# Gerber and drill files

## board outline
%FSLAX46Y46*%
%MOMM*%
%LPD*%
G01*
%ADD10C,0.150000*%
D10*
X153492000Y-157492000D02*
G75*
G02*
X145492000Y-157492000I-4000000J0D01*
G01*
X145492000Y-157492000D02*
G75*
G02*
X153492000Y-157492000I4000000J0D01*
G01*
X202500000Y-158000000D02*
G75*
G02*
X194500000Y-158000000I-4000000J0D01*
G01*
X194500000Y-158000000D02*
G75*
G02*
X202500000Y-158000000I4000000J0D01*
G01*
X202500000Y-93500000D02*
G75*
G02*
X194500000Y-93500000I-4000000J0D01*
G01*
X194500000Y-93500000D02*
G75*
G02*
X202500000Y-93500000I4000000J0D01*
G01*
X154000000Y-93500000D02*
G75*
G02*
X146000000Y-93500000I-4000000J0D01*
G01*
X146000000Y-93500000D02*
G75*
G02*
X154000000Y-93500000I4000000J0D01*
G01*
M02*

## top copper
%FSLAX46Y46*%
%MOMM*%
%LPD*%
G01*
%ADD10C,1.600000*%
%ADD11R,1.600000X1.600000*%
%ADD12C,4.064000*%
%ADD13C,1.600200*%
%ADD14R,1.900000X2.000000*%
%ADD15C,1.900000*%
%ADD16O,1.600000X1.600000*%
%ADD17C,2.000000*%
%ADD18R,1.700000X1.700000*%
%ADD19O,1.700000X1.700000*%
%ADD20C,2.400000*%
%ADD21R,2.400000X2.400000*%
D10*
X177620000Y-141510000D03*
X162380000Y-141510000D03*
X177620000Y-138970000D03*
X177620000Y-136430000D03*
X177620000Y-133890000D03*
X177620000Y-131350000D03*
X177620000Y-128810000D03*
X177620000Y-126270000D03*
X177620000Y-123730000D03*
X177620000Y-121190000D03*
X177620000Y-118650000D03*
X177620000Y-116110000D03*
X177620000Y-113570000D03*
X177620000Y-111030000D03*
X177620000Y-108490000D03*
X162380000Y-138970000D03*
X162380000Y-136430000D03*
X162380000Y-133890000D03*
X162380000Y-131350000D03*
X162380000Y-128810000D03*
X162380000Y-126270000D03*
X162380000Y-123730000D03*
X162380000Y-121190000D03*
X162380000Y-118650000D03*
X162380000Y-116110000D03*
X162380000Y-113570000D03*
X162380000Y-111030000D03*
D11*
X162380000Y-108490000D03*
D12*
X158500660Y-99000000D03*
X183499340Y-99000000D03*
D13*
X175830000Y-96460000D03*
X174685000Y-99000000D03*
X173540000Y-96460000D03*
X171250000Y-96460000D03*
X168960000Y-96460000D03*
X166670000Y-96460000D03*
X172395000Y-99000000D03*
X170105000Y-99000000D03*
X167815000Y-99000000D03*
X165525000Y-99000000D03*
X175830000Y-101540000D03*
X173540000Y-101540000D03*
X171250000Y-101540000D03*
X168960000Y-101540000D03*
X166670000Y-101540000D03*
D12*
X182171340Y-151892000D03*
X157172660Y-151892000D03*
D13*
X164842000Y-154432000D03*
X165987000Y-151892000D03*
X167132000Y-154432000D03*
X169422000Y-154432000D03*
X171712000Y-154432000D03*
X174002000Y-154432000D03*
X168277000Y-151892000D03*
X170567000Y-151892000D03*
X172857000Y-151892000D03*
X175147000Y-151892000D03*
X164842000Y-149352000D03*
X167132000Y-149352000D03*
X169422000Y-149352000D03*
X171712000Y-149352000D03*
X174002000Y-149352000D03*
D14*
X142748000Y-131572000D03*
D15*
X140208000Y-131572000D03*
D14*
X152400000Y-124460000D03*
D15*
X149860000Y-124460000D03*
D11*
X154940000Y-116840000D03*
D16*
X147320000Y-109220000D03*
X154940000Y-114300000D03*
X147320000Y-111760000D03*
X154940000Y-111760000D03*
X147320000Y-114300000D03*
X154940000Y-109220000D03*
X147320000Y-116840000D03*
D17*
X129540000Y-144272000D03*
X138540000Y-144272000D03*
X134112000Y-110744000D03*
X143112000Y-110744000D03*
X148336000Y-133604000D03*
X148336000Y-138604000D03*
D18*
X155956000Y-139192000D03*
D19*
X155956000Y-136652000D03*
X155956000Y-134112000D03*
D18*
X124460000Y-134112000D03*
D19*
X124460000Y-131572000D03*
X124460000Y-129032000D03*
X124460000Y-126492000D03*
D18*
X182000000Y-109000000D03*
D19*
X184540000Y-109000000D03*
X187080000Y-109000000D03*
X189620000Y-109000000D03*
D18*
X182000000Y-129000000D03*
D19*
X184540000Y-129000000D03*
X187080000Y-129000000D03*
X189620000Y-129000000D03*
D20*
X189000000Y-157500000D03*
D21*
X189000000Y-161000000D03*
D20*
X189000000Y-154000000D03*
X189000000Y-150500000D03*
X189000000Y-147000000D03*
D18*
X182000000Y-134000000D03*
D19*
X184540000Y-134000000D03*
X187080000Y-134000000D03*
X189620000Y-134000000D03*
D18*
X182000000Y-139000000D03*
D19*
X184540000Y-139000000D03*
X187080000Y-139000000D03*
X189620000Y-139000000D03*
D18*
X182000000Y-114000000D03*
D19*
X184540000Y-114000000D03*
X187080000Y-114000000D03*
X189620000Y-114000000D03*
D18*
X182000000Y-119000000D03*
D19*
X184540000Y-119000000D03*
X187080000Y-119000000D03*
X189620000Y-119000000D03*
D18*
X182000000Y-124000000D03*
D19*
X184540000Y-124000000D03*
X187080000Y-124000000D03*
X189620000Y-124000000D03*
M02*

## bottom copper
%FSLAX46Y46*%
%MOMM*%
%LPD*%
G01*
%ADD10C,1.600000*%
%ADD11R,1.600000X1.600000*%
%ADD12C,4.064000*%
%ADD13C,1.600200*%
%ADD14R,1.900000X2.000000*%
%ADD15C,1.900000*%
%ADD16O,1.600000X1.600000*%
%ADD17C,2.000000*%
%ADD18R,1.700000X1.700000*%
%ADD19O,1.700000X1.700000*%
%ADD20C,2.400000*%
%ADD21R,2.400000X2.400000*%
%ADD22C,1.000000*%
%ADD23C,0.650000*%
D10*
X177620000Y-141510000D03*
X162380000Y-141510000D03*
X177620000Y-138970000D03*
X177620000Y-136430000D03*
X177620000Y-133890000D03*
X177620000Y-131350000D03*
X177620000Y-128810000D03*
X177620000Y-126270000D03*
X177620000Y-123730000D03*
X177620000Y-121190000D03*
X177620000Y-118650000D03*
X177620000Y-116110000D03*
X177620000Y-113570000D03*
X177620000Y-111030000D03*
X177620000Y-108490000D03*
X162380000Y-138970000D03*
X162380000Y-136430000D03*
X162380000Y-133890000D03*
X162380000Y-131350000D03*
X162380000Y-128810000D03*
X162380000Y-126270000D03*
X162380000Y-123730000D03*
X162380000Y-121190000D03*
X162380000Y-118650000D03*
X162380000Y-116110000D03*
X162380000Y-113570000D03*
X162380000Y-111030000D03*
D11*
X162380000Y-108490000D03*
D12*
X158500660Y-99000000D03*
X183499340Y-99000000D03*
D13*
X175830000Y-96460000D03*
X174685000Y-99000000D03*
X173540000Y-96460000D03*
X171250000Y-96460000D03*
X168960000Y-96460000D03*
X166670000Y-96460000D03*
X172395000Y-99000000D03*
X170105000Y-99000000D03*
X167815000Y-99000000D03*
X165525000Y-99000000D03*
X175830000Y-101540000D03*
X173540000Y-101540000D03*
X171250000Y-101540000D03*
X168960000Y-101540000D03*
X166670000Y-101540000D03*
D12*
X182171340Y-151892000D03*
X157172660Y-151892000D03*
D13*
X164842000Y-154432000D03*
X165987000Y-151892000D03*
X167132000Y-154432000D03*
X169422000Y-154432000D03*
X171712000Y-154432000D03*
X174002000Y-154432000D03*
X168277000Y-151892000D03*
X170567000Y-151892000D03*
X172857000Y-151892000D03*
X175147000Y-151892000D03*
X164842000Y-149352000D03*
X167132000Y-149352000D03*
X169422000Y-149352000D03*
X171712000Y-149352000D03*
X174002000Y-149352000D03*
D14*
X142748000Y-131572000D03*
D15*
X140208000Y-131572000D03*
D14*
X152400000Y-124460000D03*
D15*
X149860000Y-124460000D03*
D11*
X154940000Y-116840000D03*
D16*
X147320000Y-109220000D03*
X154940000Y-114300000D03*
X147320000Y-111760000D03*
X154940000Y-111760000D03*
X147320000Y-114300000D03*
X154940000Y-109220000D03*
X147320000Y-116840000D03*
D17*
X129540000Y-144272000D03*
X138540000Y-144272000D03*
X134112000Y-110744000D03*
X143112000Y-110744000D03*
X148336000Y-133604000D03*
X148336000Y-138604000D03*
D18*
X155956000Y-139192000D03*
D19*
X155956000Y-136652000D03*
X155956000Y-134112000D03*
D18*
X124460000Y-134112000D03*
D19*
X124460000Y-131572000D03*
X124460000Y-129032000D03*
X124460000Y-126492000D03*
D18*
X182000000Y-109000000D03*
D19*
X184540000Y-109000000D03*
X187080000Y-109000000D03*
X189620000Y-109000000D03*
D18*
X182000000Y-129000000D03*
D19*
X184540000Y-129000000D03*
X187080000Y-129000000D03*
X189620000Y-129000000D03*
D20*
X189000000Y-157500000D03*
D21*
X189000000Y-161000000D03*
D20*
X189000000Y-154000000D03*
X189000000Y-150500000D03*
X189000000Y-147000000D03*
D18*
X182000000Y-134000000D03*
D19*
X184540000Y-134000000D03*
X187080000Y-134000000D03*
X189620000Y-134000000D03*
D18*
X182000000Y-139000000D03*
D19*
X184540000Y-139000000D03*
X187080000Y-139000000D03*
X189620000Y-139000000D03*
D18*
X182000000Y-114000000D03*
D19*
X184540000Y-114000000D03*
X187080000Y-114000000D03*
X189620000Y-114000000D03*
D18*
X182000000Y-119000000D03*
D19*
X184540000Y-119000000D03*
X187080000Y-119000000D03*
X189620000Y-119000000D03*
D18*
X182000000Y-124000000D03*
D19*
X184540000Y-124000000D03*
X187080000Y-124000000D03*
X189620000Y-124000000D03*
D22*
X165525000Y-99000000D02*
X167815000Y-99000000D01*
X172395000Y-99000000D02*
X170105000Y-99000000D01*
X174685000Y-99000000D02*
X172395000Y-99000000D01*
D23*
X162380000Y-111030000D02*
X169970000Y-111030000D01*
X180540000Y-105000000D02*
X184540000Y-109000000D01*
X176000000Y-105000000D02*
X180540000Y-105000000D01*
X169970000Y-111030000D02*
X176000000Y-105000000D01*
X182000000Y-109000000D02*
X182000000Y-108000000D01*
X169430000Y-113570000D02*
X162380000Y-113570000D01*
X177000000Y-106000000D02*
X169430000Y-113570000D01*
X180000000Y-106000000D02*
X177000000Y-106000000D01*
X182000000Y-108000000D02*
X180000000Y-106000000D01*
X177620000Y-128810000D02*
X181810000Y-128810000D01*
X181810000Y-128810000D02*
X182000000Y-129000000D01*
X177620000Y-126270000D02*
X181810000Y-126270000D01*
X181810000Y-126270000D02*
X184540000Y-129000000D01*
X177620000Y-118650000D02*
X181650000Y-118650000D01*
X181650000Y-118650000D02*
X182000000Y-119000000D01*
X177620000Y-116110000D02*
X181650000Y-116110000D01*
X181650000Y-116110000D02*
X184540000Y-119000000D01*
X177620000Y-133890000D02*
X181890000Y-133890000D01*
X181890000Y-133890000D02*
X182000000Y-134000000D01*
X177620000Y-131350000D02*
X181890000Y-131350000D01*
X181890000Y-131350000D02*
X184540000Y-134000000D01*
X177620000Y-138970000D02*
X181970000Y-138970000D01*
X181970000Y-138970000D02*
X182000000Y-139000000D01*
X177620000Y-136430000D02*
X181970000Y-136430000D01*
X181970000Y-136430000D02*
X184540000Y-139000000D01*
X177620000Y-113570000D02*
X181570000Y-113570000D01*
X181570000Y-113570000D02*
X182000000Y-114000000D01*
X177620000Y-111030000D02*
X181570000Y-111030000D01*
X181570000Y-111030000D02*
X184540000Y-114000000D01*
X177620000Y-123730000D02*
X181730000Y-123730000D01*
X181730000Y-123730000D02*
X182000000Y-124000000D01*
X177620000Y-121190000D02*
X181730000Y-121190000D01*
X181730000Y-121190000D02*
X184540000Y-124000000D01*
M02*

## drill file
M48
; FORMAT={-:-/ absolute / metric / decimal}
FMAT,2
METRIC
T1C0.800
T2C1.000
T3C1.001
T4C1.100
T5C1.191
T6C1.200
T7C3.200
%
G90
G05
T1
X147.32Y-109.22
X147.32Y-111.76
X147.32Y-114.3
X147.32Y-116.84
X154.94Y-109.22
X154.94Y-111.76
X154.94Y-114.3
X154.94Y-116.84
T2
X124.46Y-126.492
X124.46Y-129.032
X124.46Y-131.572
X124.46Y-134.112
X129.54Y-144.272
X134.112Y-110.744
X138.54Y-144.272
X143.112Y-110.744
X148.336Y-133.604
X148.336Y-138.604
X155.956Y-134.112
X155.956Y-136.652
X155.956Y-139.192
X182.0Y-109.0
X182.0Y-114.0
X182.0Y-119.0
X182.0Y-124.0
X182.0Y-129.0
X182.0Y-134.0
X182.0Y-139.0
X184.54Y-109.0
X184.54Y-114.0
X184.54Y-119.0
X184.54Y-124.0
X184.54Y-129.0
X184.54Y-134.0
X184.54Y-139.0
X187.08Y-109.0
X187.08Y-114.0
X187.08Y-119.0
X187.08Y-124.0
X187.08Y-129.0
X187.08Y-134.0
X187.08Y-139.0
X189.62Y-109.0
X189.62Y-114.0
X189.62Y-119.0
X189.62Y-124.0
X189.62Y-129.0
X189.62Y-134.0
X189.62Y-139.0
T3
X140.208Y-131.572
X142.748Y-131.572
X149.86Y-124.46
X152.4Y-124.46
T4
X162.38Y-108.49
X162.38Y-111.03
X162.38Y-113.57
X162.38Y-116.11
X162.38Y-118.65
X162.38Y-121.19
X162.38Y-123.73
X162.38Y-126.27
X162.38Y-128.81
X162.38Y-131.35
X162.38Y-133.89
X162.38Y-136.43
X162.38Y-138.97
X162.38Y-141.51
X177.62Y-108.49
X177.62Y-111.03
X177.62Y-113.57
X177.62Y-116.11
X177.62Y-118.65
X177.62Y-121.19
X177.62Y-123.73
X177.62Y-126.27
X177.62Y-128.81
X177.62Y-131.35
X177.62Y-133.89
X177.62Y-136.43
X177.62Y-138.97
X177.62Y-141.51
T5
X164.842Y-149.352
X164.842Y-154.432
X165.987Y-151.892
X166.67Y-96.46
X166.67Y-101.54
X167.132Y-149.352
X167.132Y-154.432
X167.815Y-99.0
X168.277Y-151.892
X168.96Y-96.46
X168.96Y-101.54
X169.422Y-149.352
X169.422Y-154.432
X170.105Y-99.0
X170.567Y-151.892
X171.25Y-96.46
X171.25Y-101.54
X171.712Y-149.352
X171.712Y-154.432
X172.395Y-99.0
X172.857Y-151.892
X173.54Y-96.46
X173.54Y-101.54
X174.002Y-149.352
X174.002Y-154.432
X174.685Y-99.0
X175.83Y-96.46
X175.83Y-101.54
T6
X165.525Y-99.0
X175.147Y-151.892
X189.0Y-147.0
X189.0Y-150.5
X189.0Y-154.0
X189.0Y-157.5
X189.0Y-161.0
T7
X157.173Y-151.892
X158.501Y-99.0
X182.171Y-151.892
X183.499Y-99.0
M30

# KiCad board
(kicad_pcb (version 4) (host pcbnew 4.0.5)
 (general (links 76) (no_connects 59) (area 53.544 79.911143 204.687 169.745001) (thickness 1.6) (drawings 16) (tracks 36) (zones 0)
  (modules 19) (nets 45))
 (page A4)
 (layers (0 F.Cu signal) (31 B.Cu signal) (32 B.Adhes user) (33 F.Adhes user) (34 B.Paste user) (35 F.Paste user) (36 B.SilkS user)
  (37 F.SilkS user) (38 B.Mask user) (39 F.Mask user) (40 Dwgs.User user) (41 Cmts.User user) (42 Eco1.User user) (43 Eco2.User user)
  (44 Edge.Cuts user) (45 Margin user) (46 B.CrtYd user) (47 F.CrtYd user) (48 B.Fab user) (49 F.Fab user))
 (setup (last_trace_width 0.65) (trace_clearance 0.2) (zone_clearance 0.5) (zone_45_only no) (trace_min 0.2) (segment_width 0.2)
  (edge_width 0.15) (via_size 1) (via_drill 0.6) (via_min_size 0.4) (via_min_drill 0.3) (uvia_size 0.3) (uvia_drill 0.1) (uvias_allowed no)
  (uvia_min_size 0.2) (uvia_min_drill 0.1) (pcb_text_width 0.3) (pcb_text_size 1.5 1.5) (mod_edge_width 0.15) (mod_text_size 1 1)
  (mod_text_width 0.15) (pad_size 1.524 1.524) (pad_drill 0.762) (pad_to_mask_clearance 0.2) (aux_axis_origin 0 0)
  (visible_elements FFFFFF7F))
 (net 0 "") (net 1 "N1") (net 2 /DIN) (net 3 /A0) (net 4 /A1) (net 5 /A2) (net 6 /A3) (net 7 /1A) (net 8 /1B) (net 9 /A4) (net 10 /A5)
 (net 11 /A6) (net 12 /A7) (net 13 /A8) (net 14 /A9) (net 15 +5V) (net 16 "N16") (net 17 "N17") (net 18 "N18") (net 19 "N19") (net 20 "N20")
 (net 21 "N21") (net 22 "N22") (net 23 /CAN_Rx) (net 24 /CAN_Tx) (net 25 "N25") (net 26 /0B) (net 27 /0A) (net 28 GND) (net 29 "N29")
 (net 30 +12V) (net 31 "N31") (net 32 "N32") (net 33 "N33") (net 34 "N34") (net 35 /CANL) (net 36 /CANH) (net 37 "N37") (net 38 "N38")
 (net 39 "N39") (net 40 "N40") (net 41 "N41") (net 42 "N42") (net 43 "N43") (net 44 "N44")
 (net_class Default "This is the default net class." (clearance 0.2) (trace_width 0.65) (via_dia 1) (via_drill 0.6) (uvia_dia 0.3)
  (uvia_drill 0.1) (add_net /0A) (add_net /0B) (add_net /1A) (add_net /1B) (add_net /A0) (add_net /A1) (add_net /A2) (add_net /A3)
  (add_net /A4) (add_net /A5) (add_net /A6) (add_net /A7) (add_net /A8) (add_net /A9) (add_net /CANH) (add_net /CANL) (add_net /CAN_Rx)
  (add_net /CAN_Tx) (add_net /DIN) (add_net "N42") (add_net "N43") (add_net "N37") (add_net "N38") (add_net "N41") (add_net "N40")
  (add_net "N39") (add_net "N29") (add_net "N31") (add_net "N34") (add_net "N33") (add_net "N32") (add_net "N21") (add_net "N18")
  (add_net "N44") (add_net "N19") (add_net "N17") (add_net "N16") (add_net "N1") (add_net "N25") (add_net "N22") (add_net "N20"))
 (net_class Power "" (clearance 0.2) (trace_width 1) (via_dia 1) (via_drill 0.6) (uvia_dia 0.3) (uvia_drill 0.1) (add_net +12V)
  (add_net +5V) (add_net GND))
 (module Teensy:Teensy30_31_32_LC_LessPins (layer F.Cu) (at 170 125 270)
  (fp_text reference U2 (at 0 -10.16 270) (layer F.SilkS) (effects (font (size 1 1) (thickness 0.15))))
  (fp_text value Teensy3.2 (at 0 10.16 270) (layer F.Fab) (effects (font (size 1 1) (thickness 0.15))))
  (pad 20 thru_hole circle (at 16.51 -7.62 270) (size 1.6 1.6) (drill 1.1) (layers *.Cu *.Mask F.SilkS) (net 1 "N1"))
  (pad 14 thru_hole circle (at 16.51 7.62 270) (size 1.6 1.6) (drill 1.1) (layers *.Cu *.Mask F.SilkS) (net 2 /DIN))
  (pad 21 thru_hole circle (at 13.97 -7.62 270) (size 1.6 1.6) (drill 1.1) (layers *.Cu *.Mask F.SilkS) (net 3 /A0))
  (pad 22 thru_hole circle (at 11.43 -7.62 270) (size 1.6 1.6) (drill 1.1) (layers *.Cu *.Mask F.SilkS) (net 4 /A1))
  (pad 23 thru_hole circle (at 8.89 -7.62 270) (size 1.6 1.6) (drill 1.1) (layers *.Cu *.Mask F.SilkS) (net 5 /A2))
  (pad 24 thru_hole circle (at 6.35 -7.62 270) (size 1.6 1.6) (drill 1.1) (layers *.Cu *.Mask F.SilkS) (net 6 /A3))
  (pad 25 thru_hole circle (at 3.81 -7.62 270) (size 1.6 1.6) (drill 1.1) (layers *.Cu *.Mask F.SilkS) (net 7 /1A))
  (pad 26 thru_hole circle (at 1.27 -7.62 270) (size 1.6 1.6) (drill 1.1) (layers *.Cu *.Mask F.SilkS) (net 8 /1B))
  (pad 27 thru_hole circle (at -1.27 -7.62 270) (size 1.6 1.6) (drill 1.1) (layers *.Cu *.Mask F.SilkS) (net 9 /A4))
  (pad 28 thru_hole circle (at -3.81 -7.62 270) (size 1.6 1.6) (drill 1.1) (layers *.Cu *.Mask F.SilkS) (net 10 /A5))
  (pad 29 thru_hole circle (at -6.35 -7.62 270) (size 1.6 1.6) (drill 1.1) (layers *.Cu *.Mask F.SilkS) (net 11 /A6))
  (pad 30 thru_hole circle (at -8.89 -7.62 270) (size 1.6 1.6) (drill 1.1) (layers *.Cu *.Mask F.SilkS) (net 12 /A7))
  (pad 31 thru_hole circle (at -11.43 -7.62 270) (size 1.6 1.6) (drill 1.1) (layers *.Cu *.Mask F.SilkS) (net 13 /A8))
  (pad 32 thru_hole circle (at -13.97 -7.62 270) (size 1.6 1.6) (drill 1.1) (layers *.Cu *.Mask F.SilkS) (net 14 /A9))
  (pad 33 thru_hole circle (at -16.51 -7.62 270) (size 1.6 1.6) (drill 1.1) (layers *.Cu *.Mask F.SilkS) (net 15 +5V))
  (pad 13 thru_hole circle (at 13.97 7.62 270) (size 1.6 1.6) (drill 1.1) (layers *.Cu *.Mask F.SilkS) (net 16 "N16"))
  (pad 12 thru_hole circle (at 11.43 7.62 270) (size 1.6 1.6) (drill 1.1) (layers *.Cu *.Mask F.SilkS) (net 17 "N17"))
  (pad 11 thru_hole circle (at 8.89 7.62 270) (size 1.6 1.6) (drill 1.1) (layers *.Cu *.Mask F.SilkS) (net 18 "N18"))
  (pad 10 thru_hole circle (at 6.35 7.62 270) (size 1.6 1.6) (drill 1.1) (layers *.Cu *.Mask F.SilkS) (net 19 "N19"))
  (pad 9 thru_hole circle (at 3.81 7.62 270) (size 1.6 1.6) (drill 1.1) (layers *.Cu *.Mask F.SilkS) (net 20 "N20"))
  (pad 8 thru_hole circle (at 1.27 7.62 270) (size 1.6 1.6) (drill 1.1) (layers *.Cu *.Mask F.SilkS) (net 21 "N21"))
  (pad 7 thru_hole circle (at -1.27 7.62 270) (size 1.6 1.6) (drill 1.1) (layers *.Cu *.Mask F.SilkS) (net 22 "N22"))
  (pad 6 thru_hole circle (at -3.81 7.62 270) (size 1.6 1.6) (drill 1.1) (layers *.Cu *.Mask F.SilkS) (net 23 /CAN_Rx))
  (pad 5 thru_hole circle (at -6.35 7.62 270) (size 1.6 1.6) (drill 1.1) (layers *.Cu *.Mask F.SilkS) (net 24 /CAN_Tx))
  (pad 4 thru_hole circle (at -8.89 7.62 270) (size 1.6 1.6) (drill 1.1) (layers *.Cu *.Mask F.SilkS) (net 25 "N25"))
  (pad 3 thru_hole circle (at -11.43 7.62 270) (size 1.6 1.6) (drill 1.1) (layers *.Cu *.Mask F.SilkS) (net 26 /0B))
  (pad 2 thru_hole circle (at -13.97 7.62 270) (size 1.6 1.6) (drill 1.1) (layers *.Cu *.Mask F.SilkS) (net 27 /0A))
  (pad 1 thru_hole rect (at -16.51 7.62 270) (size 1.6 1.6) (drill 1.1) (layers *.Cu *.Mask F.SilkS) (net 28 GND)))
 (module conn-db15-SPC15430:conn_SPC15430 (layer F.Cu) (at 171 99)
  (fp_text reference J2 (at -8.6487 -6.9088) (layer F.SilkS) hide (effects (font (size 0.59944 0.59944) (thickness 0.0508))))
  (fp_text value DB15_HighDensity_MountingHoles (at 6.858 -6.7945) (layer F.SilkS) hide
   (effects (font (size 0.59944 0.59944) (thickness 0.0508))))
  (pad 0 thru_hole circle (at -12.49934 0) (size 4.064 4.064) (drill 3.2004) (layers *.Cu *.Mask) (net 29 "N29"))
  (pad 0 thru_hole circle (at 12.49934 0) (size 4.064 4.064) (drill 3.2004) (layers *.Cu *.Mask) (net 29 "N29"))
  (pad 15 thru_hole circle (at 4.83 -2.54) (size 1.6002 1.6002) (drill 1.19126) (layers *.Cu *.Mask) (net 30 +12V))
  (pad 10 thru_hole circle (at 3.685 0) (size 1.6002 1.6002) (drill 1.19126) (layers *.Cu *.Mask) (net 28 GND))
  (pad 14 thru_hole circle (at 2.54 -2.54) (size 1.6002 1.6002) (drill 1.19126) (layers *.Cu *.Mask) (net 30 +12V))
  (pad 13 thru_hole circle (at 0.25 -2.54) (size 1.6002 1.6002) (drill 1.19126) (layers *.Cu *.Mask) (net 15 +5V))
  (pad 12 thru_hole circle (at -2.04 -2.54) (size 1.6002 1.6002) (drill 1.19126) (layers *.Cu *.Mask) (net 15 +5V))
  (pad 11 thru_hole circle (at -4.33 -2.54) (size 1.6002 1.6002) (drill 1.19126) (layers *.Cu *.Mask) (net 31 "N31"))
  (pad 9 thru_hole circle (at 1.395 0) (size 1.6002 1.6002) (drill 1.19126) (layers *.Cu *.Mask) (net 28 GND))
  (pad 8 thru_hole circle (at -0.895 0) (size 1.6002 1.6002) (drill 1.19126) (layers *.Cu *.Mask) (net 28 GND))
  (pad 7 thru_hole circle (at -3.185 0) (size 1.6002 1.6002) (drill 1.19126) (layers *.Cu *.Mask) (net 28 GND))
  (pad 6 thru_hole circle (at -5.475 0) (size 1.6002 1.6002) (drill 1.2) (layers *.Cu *.Mask) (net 28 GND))
  (pad 5 thru_hole circle (at 4.83 2.54) (size 1.6002 1.6002) (drill 1.19126) (layers *.Cu *.Mask) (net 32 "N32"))
  (pad 4 thru_hole circle (at 2.54 2.54) (size 1.6002 1.6002) (drill 1.19126) (layers *.Cu *.Mask) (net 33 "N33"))
  (pad 3 thru_hole circle (at 0.25 2.54) (size 1.6002 1.6002) (drill 1.19126) (layers *.Cu *.Mask) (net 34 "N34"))
  (pad 2 thru_hole circle (at -2.04 2.54) (size 1.6002 1.6002) (drill 1.19126) (layers *.Cu *.Mask) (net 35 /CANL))
  (pad 1 thru_hole circle (at -4.33 2.54) (size 1.6002 1.6002) (drill 1.19126) (layers *.Cu *.Mask) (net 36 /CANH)))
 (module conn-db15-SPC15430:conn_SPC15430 (layer F.Cu) (at 169.672 151.892 180)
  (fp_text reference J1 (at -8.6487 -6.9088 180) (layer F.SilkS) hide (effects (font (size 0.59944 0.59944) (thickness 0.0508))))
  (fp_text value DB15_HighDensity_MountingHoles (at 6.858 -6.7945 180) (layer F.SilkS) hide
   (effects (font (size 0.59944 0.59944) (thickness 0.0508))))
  (pad 0 thru_hole circle (at -12.49934 0 180) (size 4.064 4.064) (drill 3.2004) (layers *.Cu *.Mask) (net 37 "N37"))
  (pad 0 thru_hole circle (at 12.49934 0 180) (size 4.064 4.064) (drill 3.2004) (layers *.Cu *.Mask) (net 37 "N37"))
  (pad 15 thru_hole circle (at 4.83 -2.54 180) (size 1.6002 1.6002) (drill 1.19126) (layers *.Cu *.Mask) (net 30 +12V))
  (pad 10 thru_hole circle (at 3.685 0 180) (size 1.6002 1.6002) (drill 1.19126) (layers *.Cu *.Mask) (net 28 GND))
  (pad 14 thru_hole circle (at 2.54 -2.54 180) (size 1.6002 1.6002) (drill 1.19126) (layers *.Cu *.Mask) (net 30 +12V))
  (pad 13 thru_hole circle (at 0.25 -2.54 180) (size 1.6002 1.6002) (drill 1.19126) (layers *.Cu *.Mask) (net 15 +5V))
  (pad 12 thru_hole circle (at -2.04 -2.54 180) (size 1.6002 1.6002) (drill 1.19126) (layers *.Cu *.Mask) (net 15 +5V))
  (pad 11 thru_hole circle (at -4.33 -2.54 180) (size 1.6002 1.6002) (drill 1.19126) (layers *.Cu *.Mask) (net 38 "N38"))
  (pad 9 thru_hole circle (at 1.395 0 180) (size 1.6002 1.6002) (drill 1.19126) (layers *.Cu *.Mask) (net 28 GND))
  (pad 8 thru_hole circle (at -0.895 0 180) (size 1.6002 1.6002) (drill 1.19126) (layers *.Cu *.Mask) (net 28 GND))
  (pad 7 thru_hole circle (at -3.185 0 180) (size 1.6002 1.6002) (drill 1.19126) (layers *.Cu *.Mask) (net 28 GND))
  (pad 6 thru_hole circle (at -5.475 0 180) (size 1.6002 1.6002) (drill 1.2) (layers *.Cu *.Mask) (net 28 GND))
  (pad 5 thru_hole circle (at 4.83 2.54 180) (size 1.6002 1.6002) (drill 1.19126) (layers *.Cu *.Mask) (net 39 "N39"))
  (pad 4 thru_hole circle (at 2.54 2.54 180) (size 1.6002 1.6002) (drill 1.19126) (layers *.Cu *.Mask) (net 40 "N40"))
  (pad 3 thru_hole circle (at 0.25 2.54 180) (size 1.6002 1.6002) (drill 1.19126) (layers *.Cu *.Mask) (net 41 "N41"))
  (pad 2 thru_hole circle (at -2.04 2.54 180) (size 1.6002 1.6002) (drill 1.19126) (layers *.Cu *.Mask) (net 35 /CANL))
  (pad 1 thru_hole circle (at -4.33 2.54 180) (size 1.6002 1.6002) (drill 1.19126) (layers *.Cu *.Mask) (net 36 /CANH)))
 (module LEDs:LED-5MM (layer F.Cu) (at 142.748 131.572 180)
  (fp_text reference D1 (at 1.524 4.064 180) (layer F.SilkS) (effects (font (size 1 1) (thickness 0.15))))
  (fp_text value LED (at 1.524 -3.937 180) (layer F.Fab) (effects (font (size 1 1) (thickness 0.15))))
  (pad 1 thru_hole rect (at 0 0 270) (size 2 1.9) (drill 1.00076) (layers *.Cu *.Mask) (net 28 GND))
  (pad 2 thru_hole circle (at 2.54 0 180) (size 1.9 1.9) (drill 1.00076) (layers *.Cu *.Mask) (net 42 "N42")))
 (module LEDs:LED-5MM (layer F.Cu) (at 152.4 124.46 180)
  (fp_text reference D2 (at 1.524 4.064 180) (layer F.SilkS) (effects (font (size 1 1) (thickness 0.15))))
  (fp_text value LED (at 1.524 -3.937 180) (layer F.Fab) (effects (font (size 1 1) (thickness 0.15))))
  (pad 1 thru_hole rect (at 0 0 270) (size 2 1.9) (drill 1.00076) (layers *.Cu *.Mask) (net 28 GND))
  (pad 2 thru_hole circle (at 2.54 0 180) (size 1.9 1.9) (drill 1.00076) (layers *.Cu *.Mask) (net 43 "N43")))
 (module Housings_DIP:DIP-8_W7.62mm (layer F.Cu) (at 154.94 116.84 180)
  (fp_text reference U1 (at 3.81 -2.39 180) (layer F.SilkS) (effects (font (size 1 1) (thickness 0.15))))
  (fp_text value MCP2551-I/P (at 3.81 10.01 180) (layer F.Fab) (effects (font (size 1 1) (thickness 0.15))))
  (pad 1 thru_hole rect (at 0 0 180) (size 1.6 1.6) (drill 0.8) (layers *.Cu *.Mask) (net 24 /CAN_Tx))
  (pad 5 thru_hole oval (at 7.62 7.62 180) (size 1.6 1.6) (drill 0.8) (layers *.Cu *.Mask) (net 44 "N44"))
  (pad 2 thru_hole oval (at 0 2.54 180) (size 1.6 1.6) (drill 0.8) (layers *.Cu *.Mask) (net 28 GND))
  (pad 6 thru_hole oval (at 7.62 5.08 180) (size 1.6 1.6) (drill 0.8) (layers *.Cu *.Mask) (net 35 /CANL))
  (pad 3 thru_hole oval (at 0 5.08 180) (size 1.6 1.6) (drill 0.8) (layers *.Cu *.Mask) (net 15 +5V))
  (pad 7 thru_hole oval (at 7.62 2.54 180) (size 1.6 1.6) (drill 0.8) (layers *.Cu *.Mask) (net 36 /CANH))
  (pad 4 thru_hole oval (at 0 7.62 180) (size 1.6 1.6) (drill 0.8) (layers *.Cu *.Mask) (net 23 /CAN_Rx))
  (pad 8 thru_hole oval (at 7.62 0 180) (size 1.6 1.6) (drill 0.8) (layers *.Cu *.Mask) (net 28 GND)))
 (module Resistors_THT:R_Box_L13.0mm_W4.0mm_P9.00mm (layer F.Cu) (at 129.54 144.272)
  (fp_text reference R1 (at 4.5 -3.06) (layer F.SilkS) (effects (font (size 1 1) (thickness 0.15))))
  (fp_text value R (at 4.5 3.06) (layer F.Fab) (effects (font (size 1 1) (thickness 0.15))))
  (pad 1 thru_hole circle (at 0 0) (size 2 2) (drill 1) (layers *.Cu *.Mask) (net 21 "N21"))
  (pad 2 thru_hole circle (at 9 0) (size 2 2) (drill 1) (layers *.Cu *.Mask) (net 42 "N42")))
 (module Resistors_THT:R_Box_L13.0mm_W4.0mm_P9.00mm (layer F.Cu) (at 134.112 110.744)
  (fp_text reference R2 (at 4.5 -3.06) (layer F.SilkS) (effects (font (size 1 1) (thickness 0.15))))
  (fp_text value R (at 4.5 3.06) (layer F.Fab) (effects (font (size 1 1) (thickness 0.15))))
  (pad 1 thru_hole circle (at 0 0) (size 2 2) (drill 1) (layers *.Cu *.Mask) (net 18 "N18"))
  (pad 2 thru_hole circle (at 9 0) (size 2 2) (drill 1) (layers *.Cu *.Mask) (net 43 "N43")))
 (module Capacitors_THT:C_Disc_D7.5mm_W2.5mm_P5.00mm (layer F.Cu) (at 148.336 133.604 270)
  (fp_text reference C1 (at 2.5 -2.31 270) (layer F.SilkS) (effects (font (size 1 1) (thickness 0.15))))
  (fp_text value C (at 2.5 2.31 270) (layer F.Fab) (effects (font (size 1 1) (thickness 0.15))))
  (pad 1 thru_hole circle (at 0 0 270) (size 2 2) (drill 1) (layers *.Cu *.Mask) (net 15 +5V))
  (pad 2 thru_hole circle (at 5 0 270) (size 2 2) (drill 1) (layers *.Cu *.Mask) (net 28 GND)))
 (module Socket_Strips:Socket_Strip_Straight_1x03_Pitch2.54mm (layer F.Cu) (at 155.956 139.192 180)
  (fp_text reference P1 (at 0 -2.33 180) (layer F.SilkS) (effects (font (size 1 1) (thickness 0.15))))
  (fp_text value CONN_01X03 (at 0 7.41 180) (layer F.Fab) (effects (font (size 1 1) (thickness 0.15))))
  (pad 1 thru_hole rect (at 0 0 180) (size 1.7 1.7) (drill 1) (layers *.Cu *.Mask) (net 28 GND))
  (pad 2 thru_hole oval (at 0 2.54 180) (size 1.7 1.7) (drill 1) (layers *.Cu *.Mask) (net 2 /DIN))
  (pad 3 thru_hole oval (at 0 5.08 180) (size 1.7 1.7) (drill 1) (layers *.Cu *.Mask) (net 15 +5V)))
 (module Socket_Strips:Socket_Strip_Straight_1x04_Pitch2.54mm (layer F.Cu) (at 124.46 134.112 180)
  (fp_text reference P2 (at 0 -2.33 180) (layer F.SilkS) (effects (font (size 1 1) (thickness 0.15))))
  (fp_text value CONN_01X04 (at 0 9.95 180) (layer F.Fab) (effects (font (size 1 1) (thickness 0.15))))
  (pad 1 thru_hole rect (at 0 0 180) (size 1.7 1.7) (drill 1) (layers *.Cu *.Mask) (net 30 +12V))
  (pad 2 thru_hole oval (at 0 2.54 180) (size 1.7 1.7) (drill 1) (layers *.Cu *.Mask) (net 28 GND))
  (pad 3 thru_hole oval (at 0 5.08 180) (size 1.7 1.7) (drill 1) (layers *.Cu *.Mask) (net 28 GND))
  (pad 4 thru_hole oval (at 0 7.62 180) (size 1.7 1.7) (drill 1) (layers *.Cu *.Mask) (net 15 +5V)))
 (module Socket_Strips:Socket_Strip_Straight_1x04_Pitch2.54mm (layer F.Cu) (at 182 109 90)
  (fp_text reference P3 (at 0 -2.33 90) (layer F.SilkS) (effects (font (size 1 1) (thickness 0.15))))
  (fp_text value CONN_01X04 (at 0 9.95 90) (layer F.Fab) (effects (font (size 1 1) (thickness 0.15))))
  (pad 1 thru_hole rect (at 0 0 90) (size 1.7 1.7) (drill 1) (layers *.Cu *.Mask) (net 26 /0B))
  (pad 2 thru_hole oval (at 0 2.54 90) (size 1.7 1.7) (drill 1) (layers *.Cu *.Mask) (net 27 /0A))
  (pad 3 thru_hole oval (at 0 5.08 90) (size 1.7 1.7) (drill 1) (layers *.Cu *.Mask) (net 15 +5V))
  (pad 4 thru_hole oval (at 0 7.62 90) (size 1.7 1.7) (drill 1) (layers *.Cu *.Mask) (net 28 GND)))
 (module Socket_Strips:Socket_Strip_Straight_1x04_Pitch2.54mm (layer F.Cu) (at 182 129 90)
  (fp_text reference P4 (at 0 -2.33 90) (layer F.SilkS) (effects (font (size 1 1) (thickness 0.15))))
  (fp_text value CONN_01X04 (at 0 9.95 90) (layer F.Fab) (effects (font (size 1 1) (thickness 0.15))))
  (pad 1 thru_hole rect (at 0 0 90) (size 1.7 1.7) (drill 1) (layers *.Cu *.Mask) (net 7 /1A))
  (pad 2 thru_hole oval (at 0 2.54 90) (size 1.7 1.7) (drill 1) (layers *.Cu *.Mask) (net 8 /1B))
  (pad 3 thru_hole oval (at 0 5.08 90) (size 1.7 1.7) (drill 1) (layers *.Cu *.Mask) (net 15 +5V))
  (pad 4 thru_hole oval (at 0 7.62 90) (size 1.7 1.7) (drill 1) (layers *.Cu *.Mask) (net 28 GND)))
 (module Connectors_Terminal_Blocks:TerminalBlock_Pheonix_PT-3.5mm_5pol (layer F.Cu) (at 189 161 90)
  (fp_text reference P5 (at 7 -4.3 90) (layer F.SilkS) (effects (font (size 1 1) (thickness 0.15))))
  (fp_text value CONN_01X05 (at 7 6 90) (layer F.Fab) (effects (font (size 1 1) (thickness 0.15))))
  (pad 2 thru_hole circle (at 3.5 0 90) (size 2.4 2.4) (drill 1.2) (layers *.Cu *.Mask) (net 36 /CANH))
  (pad 1 thru_hole rect (at 0 0 90) (size 2.4 2.4) (drill 1.2) (layers *.Cu *.Mask) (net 35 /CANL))
  (pad 3 thru_hole circle (at 7 0 90) (size 2.4 2.4) (drill 1.2) (layers *.Cu *.Mask) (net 30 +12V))
  (pad 4 thru_hole circle (at 10.5 0 90) (size 2.4 2.4) (drill 1.2) (layers *.Cu *.Mask) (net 15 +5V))
  (pad 5 thru_hole circle (at 14 0 90) (size 2.4 2.4) (drill 1.2) (layers *.Cu *.Mask) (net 28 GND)))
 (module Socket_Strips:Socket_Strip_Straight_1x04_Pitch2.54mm (layer F.Cu) (at 182 134 90)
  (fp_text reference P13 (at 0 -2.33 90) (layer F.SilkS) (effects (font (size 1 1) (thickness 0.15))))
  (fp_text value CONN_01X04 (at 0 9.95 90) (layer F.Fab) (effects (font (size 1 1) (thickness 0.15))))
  (pad 1 thru_hole rect (at 0 0 90) (size 1.7 1.7) (drill 1) (layers *.Cu *.Mask) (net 5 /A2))
  (pad 2 thru_hole oval (at 0 2.54 90) (size 1.7 1.7) (drill 1) (layers *.Cu *.Mask) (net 6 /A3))
  (pad 3 thru_hole oval (at 0 5.08 90) (size 1.7 1.7) (drill 1) (layers *.Cu *.Mask) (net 15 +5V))
  (pad 4 thru_hole oval (at 0 7.62 90) (size 1.7 1.7) (drill 1) (layers *.Cu *.Mask) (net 28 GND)))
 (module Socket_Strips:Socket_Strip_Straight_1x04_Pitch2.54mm (layer F.Cu) (at 182 139 90)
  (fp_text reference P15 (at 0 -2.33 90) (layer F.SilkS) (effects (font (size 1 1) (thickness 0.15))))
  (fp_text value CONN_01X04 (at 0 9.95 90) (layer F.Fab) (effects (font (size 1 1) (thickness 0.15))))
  (pad 1 thru_hole rect (at 0 0 90) (size 1.7 1.7) (drill 1) (layers *.Cu *.Mask) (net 3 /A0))
  (pad 2 thru_hole oval (at 0 2.54 90) (size 1.7 1.7) (drill 1) (layers *.Cu *.Mask) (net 4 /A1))
  (pad 3 thru_hole oval (at 0 5.08 90) (size 1.7 1.7) (drill 1) (layers *.Cu *.Mask) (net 15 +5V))
  (pad 4 thru_hole oval (at 0 7.62 90) (size 1.7 1.7) (drill 1) (layers *.Cu *.Mask) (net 28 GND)))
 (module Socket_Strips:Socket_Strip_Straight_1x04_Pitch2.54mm (layer F.Cu) (at 182 114 90)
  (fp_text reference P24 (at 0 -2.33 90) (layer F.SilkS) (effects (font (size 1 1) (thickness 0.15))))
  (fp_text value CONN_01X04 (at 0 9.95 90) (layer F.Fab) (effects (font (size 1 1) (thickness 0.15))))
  (pad 1 thru_hole rect (at 0 0 90) (size 1.7 1.7) (drill 1) (layers *.Cu *.Mask) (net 13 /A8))
  (pad 2 thru_hole oval (at 0 2.54 90) (size 1.7 1.7) (drill 1) (layers *.Cu *.Mask) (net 14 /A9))
  (pad 3 thru_hole oval (at 0 5.08 90) (size 1.7 1.7) (drill 1) (layers *.Cu *.Mask) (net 15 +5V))
  (pad 4 thru_hole oval (at 0 7.62 90) (size 1.7 1.7) (drill 1) (layers *.Cu *.Mask) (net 28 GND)))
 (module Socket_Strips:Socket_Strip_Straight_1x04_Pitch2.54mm (layer F.Cu) (at 182 119 90)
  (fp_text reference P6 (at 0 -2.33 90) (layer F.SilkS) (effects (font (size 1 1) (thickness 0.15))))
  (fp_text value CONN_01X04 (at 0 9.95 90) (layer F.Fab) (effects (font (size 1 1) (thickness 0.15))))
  (pad 1 thru_hole rect (at 0 0 90) (size 1.7 1.7) (drill 1) (layers *.Cu *.Mask) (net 11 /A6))
  (pad 2 thru_hole oval (at 0 2.54 90) (size 1.7 1.7) (drill 1) (layers *.Cu *.Mask) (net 12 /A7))
  (pad 3 thru_hole oval (at 0 5.08 90) (size 1.7 1.7) (drill 1) (layers *.Cu *.Mask) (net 15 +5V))
  (pad 4 thru_hole oval (at 0 7.62 90) (size 1.7 1.7) (drill 1) (layers *.Cu *.Mask) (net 28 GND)))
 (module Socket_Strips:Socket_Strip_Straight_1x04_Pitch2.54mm (layer F.Cu) (at 182 124 90)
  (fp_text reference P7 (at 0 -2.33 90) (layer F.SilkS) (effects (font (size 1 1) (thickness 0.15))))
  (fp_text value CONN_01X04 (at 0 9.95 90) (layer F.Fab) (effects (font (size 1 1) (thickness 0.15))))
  (pad 1 thru_hole rect (at 0 0 90) (size 1.7 1.7) (drill 1) (layers *.Cu *.Mask) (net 9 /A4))
  (pad 2 thru_hole oval (at 0 2.54 90) (size 1.7 1.7) (drill 1) (layers *.Cu *.Mask) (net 10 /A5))
  (pad 3 thru_hole oval (at 0 5.08 90) (size 1.7 1.7) (drill 1) (layers *.Cu *.Mask) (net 15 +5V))
  (pad 4 thru_hole oval (at 0 7.62 90) (size 1.7 1.7) (drill 1) (layers *.Cu *.Mask) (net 28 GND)))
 (gr_circle (center 149.492 157.492) (end 153.492 157.492) (layer Edge.Cuts) (width 0.15))
 (gr_circle (center 198.5 158) (end 194.5 158) (layer Edge.Cuts) (width 0.15))
 (gr_circle (center 198.5 93.5) (end 194.5 93.5) (layer Edge.Cuts) (width 0.15))
 (gr_circle (center 150 93.5) (end 154 93.5) (layer Edge.Cuts) (width 0.15))
 (segment (start 165.525 99) (end 167.815 99) (width 1) (layer B.Cu) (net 28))
 (segment (start 172.395 99) (end 170.105 99) (width 1) (layer B.Cu) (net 28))
 (segment (start 174.685 99) (end 172.395 99) (width 1) (layer B.Cu) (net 28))
 (segment (start 162.38 111.03) (end 169.97 111.03) (width 0.65) (layer B.Cu) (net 27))
 (segment (start 180.54 105) (end 184.54 109) (width 0.65) (layer B.Cu) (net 27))
 (segment (start 176 105) (end 180.54 105) (width 0.65) (layer B.Cu) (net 27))
 (segment (start 169.97 111.03) (end 176 105) (width 0.65) (layer B.Cu) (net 27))
 (segment (start 182 109) (end 182 108) (width 0.65) (layer B.Cu) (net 26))
 (segment (start 169.43 113.57) (end 162.38 113.57) (width 0.65) (layer B.Cu) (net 26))
 (segment (start 177 106) (end 169.43 113.57) (width 0.65) (layer B.Cu) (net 26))
 (segment (start 180 106) (end 177 106) (width 0.65) (layer B.Cu) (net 26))
 (segment (start 182 108) (end 180 106) (width 0.65) (layer B.Cu) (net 26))
 (segment (start 177.62 128.81) (end 181.81 128.81) (width 0.65) (layer B.Cu) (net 7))
 (segment (start 181.81 128.81) (end 182 129) (width 0.65) (layer B.Cu) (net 7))
 (segment (start 177.62 126.27) (end 181.81 126.27) (width 0.65) (layer B.Cu) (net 8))
 (segment (start 181.81 126.27) (end 184.54 129) (width 0.65) (layer B.Cu) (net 8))
 (segment (start 177.62 118.65) (end 181.65 118.65) (width 0.65) (layer B.Cu) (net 11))
 (segment (start 181.65 118.65) (end 182 119) (width 0.65) (layer B.Cu) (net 11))
 (segment (start 177.62 116.11) (end 181.65 116.11) (width 0.65) (layer B.Cu) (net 12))
 (segment (start 181.65 116.11) (end 184.54 119) (width 0.65) (layer B.Cu) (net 12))
 (segment (start 177.62 133.89) (end 181.89 133.89) (width 0.65) (layer B.Cu) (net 5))
 (segment (start 181.89 133.89) (end 182 134) (width 0.65) (layer B.Cu) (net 5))
 (segment (start 177.62 131.35) (end 181.89 131.35) (width 0.65) (layer B.Cu) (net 6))
 (segment (start 181.89 131.35) (end 184.54 134) (width 0.65) (layer B.Cu) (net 6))
 (segment (start 177.62 138.97) (end 181.97 138.97) (width 0.65) (layer B.Cu) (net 3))
 (segment (start 181.97 138.97) (end 182 139) (width 0.65) (layer B.Cu) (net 3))
 (segment (start 177.62 136.43) (end 181.97 136.43) (width 0.65) (layer B.Cu) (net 4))
 (segment (start 181.97 136.43) (end 184.54 139) (width 0.65) (layer B.Cu) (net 4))
 (segment (start 177.62 113.57) (end 181.57 113.57) (width 0.65) (layer B.Cu) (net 13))
 (segment (start 181.57 113.57) (end 182 114) (width 0.65) (layer B.Cu) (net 13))
 (segment (start 177.62 111.03) (end 181.57 111.03) (width 0.65) (layer B.Cu) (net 14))
 (segment (start 181.57 111.03) (end 184.54 114) (width 0.65) (layer B.Cu) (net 14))
 (segment (start 177.62 123.73) (end 181.73 123.73) (width 0.65) (layer B.Cu) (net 9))
 (segment (start 181.73 123.73) (end 182 124) (width 0.65) (layer B.Cu) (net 9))
 (segment (start 177.62 121.19) (end 181.73 121.19) (width 0.65) (layer B.Cu) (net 10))
 (segment (start 181.73 121.19) (end 184.54 124) (width 0.65) (layer B.Cu) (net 10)))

